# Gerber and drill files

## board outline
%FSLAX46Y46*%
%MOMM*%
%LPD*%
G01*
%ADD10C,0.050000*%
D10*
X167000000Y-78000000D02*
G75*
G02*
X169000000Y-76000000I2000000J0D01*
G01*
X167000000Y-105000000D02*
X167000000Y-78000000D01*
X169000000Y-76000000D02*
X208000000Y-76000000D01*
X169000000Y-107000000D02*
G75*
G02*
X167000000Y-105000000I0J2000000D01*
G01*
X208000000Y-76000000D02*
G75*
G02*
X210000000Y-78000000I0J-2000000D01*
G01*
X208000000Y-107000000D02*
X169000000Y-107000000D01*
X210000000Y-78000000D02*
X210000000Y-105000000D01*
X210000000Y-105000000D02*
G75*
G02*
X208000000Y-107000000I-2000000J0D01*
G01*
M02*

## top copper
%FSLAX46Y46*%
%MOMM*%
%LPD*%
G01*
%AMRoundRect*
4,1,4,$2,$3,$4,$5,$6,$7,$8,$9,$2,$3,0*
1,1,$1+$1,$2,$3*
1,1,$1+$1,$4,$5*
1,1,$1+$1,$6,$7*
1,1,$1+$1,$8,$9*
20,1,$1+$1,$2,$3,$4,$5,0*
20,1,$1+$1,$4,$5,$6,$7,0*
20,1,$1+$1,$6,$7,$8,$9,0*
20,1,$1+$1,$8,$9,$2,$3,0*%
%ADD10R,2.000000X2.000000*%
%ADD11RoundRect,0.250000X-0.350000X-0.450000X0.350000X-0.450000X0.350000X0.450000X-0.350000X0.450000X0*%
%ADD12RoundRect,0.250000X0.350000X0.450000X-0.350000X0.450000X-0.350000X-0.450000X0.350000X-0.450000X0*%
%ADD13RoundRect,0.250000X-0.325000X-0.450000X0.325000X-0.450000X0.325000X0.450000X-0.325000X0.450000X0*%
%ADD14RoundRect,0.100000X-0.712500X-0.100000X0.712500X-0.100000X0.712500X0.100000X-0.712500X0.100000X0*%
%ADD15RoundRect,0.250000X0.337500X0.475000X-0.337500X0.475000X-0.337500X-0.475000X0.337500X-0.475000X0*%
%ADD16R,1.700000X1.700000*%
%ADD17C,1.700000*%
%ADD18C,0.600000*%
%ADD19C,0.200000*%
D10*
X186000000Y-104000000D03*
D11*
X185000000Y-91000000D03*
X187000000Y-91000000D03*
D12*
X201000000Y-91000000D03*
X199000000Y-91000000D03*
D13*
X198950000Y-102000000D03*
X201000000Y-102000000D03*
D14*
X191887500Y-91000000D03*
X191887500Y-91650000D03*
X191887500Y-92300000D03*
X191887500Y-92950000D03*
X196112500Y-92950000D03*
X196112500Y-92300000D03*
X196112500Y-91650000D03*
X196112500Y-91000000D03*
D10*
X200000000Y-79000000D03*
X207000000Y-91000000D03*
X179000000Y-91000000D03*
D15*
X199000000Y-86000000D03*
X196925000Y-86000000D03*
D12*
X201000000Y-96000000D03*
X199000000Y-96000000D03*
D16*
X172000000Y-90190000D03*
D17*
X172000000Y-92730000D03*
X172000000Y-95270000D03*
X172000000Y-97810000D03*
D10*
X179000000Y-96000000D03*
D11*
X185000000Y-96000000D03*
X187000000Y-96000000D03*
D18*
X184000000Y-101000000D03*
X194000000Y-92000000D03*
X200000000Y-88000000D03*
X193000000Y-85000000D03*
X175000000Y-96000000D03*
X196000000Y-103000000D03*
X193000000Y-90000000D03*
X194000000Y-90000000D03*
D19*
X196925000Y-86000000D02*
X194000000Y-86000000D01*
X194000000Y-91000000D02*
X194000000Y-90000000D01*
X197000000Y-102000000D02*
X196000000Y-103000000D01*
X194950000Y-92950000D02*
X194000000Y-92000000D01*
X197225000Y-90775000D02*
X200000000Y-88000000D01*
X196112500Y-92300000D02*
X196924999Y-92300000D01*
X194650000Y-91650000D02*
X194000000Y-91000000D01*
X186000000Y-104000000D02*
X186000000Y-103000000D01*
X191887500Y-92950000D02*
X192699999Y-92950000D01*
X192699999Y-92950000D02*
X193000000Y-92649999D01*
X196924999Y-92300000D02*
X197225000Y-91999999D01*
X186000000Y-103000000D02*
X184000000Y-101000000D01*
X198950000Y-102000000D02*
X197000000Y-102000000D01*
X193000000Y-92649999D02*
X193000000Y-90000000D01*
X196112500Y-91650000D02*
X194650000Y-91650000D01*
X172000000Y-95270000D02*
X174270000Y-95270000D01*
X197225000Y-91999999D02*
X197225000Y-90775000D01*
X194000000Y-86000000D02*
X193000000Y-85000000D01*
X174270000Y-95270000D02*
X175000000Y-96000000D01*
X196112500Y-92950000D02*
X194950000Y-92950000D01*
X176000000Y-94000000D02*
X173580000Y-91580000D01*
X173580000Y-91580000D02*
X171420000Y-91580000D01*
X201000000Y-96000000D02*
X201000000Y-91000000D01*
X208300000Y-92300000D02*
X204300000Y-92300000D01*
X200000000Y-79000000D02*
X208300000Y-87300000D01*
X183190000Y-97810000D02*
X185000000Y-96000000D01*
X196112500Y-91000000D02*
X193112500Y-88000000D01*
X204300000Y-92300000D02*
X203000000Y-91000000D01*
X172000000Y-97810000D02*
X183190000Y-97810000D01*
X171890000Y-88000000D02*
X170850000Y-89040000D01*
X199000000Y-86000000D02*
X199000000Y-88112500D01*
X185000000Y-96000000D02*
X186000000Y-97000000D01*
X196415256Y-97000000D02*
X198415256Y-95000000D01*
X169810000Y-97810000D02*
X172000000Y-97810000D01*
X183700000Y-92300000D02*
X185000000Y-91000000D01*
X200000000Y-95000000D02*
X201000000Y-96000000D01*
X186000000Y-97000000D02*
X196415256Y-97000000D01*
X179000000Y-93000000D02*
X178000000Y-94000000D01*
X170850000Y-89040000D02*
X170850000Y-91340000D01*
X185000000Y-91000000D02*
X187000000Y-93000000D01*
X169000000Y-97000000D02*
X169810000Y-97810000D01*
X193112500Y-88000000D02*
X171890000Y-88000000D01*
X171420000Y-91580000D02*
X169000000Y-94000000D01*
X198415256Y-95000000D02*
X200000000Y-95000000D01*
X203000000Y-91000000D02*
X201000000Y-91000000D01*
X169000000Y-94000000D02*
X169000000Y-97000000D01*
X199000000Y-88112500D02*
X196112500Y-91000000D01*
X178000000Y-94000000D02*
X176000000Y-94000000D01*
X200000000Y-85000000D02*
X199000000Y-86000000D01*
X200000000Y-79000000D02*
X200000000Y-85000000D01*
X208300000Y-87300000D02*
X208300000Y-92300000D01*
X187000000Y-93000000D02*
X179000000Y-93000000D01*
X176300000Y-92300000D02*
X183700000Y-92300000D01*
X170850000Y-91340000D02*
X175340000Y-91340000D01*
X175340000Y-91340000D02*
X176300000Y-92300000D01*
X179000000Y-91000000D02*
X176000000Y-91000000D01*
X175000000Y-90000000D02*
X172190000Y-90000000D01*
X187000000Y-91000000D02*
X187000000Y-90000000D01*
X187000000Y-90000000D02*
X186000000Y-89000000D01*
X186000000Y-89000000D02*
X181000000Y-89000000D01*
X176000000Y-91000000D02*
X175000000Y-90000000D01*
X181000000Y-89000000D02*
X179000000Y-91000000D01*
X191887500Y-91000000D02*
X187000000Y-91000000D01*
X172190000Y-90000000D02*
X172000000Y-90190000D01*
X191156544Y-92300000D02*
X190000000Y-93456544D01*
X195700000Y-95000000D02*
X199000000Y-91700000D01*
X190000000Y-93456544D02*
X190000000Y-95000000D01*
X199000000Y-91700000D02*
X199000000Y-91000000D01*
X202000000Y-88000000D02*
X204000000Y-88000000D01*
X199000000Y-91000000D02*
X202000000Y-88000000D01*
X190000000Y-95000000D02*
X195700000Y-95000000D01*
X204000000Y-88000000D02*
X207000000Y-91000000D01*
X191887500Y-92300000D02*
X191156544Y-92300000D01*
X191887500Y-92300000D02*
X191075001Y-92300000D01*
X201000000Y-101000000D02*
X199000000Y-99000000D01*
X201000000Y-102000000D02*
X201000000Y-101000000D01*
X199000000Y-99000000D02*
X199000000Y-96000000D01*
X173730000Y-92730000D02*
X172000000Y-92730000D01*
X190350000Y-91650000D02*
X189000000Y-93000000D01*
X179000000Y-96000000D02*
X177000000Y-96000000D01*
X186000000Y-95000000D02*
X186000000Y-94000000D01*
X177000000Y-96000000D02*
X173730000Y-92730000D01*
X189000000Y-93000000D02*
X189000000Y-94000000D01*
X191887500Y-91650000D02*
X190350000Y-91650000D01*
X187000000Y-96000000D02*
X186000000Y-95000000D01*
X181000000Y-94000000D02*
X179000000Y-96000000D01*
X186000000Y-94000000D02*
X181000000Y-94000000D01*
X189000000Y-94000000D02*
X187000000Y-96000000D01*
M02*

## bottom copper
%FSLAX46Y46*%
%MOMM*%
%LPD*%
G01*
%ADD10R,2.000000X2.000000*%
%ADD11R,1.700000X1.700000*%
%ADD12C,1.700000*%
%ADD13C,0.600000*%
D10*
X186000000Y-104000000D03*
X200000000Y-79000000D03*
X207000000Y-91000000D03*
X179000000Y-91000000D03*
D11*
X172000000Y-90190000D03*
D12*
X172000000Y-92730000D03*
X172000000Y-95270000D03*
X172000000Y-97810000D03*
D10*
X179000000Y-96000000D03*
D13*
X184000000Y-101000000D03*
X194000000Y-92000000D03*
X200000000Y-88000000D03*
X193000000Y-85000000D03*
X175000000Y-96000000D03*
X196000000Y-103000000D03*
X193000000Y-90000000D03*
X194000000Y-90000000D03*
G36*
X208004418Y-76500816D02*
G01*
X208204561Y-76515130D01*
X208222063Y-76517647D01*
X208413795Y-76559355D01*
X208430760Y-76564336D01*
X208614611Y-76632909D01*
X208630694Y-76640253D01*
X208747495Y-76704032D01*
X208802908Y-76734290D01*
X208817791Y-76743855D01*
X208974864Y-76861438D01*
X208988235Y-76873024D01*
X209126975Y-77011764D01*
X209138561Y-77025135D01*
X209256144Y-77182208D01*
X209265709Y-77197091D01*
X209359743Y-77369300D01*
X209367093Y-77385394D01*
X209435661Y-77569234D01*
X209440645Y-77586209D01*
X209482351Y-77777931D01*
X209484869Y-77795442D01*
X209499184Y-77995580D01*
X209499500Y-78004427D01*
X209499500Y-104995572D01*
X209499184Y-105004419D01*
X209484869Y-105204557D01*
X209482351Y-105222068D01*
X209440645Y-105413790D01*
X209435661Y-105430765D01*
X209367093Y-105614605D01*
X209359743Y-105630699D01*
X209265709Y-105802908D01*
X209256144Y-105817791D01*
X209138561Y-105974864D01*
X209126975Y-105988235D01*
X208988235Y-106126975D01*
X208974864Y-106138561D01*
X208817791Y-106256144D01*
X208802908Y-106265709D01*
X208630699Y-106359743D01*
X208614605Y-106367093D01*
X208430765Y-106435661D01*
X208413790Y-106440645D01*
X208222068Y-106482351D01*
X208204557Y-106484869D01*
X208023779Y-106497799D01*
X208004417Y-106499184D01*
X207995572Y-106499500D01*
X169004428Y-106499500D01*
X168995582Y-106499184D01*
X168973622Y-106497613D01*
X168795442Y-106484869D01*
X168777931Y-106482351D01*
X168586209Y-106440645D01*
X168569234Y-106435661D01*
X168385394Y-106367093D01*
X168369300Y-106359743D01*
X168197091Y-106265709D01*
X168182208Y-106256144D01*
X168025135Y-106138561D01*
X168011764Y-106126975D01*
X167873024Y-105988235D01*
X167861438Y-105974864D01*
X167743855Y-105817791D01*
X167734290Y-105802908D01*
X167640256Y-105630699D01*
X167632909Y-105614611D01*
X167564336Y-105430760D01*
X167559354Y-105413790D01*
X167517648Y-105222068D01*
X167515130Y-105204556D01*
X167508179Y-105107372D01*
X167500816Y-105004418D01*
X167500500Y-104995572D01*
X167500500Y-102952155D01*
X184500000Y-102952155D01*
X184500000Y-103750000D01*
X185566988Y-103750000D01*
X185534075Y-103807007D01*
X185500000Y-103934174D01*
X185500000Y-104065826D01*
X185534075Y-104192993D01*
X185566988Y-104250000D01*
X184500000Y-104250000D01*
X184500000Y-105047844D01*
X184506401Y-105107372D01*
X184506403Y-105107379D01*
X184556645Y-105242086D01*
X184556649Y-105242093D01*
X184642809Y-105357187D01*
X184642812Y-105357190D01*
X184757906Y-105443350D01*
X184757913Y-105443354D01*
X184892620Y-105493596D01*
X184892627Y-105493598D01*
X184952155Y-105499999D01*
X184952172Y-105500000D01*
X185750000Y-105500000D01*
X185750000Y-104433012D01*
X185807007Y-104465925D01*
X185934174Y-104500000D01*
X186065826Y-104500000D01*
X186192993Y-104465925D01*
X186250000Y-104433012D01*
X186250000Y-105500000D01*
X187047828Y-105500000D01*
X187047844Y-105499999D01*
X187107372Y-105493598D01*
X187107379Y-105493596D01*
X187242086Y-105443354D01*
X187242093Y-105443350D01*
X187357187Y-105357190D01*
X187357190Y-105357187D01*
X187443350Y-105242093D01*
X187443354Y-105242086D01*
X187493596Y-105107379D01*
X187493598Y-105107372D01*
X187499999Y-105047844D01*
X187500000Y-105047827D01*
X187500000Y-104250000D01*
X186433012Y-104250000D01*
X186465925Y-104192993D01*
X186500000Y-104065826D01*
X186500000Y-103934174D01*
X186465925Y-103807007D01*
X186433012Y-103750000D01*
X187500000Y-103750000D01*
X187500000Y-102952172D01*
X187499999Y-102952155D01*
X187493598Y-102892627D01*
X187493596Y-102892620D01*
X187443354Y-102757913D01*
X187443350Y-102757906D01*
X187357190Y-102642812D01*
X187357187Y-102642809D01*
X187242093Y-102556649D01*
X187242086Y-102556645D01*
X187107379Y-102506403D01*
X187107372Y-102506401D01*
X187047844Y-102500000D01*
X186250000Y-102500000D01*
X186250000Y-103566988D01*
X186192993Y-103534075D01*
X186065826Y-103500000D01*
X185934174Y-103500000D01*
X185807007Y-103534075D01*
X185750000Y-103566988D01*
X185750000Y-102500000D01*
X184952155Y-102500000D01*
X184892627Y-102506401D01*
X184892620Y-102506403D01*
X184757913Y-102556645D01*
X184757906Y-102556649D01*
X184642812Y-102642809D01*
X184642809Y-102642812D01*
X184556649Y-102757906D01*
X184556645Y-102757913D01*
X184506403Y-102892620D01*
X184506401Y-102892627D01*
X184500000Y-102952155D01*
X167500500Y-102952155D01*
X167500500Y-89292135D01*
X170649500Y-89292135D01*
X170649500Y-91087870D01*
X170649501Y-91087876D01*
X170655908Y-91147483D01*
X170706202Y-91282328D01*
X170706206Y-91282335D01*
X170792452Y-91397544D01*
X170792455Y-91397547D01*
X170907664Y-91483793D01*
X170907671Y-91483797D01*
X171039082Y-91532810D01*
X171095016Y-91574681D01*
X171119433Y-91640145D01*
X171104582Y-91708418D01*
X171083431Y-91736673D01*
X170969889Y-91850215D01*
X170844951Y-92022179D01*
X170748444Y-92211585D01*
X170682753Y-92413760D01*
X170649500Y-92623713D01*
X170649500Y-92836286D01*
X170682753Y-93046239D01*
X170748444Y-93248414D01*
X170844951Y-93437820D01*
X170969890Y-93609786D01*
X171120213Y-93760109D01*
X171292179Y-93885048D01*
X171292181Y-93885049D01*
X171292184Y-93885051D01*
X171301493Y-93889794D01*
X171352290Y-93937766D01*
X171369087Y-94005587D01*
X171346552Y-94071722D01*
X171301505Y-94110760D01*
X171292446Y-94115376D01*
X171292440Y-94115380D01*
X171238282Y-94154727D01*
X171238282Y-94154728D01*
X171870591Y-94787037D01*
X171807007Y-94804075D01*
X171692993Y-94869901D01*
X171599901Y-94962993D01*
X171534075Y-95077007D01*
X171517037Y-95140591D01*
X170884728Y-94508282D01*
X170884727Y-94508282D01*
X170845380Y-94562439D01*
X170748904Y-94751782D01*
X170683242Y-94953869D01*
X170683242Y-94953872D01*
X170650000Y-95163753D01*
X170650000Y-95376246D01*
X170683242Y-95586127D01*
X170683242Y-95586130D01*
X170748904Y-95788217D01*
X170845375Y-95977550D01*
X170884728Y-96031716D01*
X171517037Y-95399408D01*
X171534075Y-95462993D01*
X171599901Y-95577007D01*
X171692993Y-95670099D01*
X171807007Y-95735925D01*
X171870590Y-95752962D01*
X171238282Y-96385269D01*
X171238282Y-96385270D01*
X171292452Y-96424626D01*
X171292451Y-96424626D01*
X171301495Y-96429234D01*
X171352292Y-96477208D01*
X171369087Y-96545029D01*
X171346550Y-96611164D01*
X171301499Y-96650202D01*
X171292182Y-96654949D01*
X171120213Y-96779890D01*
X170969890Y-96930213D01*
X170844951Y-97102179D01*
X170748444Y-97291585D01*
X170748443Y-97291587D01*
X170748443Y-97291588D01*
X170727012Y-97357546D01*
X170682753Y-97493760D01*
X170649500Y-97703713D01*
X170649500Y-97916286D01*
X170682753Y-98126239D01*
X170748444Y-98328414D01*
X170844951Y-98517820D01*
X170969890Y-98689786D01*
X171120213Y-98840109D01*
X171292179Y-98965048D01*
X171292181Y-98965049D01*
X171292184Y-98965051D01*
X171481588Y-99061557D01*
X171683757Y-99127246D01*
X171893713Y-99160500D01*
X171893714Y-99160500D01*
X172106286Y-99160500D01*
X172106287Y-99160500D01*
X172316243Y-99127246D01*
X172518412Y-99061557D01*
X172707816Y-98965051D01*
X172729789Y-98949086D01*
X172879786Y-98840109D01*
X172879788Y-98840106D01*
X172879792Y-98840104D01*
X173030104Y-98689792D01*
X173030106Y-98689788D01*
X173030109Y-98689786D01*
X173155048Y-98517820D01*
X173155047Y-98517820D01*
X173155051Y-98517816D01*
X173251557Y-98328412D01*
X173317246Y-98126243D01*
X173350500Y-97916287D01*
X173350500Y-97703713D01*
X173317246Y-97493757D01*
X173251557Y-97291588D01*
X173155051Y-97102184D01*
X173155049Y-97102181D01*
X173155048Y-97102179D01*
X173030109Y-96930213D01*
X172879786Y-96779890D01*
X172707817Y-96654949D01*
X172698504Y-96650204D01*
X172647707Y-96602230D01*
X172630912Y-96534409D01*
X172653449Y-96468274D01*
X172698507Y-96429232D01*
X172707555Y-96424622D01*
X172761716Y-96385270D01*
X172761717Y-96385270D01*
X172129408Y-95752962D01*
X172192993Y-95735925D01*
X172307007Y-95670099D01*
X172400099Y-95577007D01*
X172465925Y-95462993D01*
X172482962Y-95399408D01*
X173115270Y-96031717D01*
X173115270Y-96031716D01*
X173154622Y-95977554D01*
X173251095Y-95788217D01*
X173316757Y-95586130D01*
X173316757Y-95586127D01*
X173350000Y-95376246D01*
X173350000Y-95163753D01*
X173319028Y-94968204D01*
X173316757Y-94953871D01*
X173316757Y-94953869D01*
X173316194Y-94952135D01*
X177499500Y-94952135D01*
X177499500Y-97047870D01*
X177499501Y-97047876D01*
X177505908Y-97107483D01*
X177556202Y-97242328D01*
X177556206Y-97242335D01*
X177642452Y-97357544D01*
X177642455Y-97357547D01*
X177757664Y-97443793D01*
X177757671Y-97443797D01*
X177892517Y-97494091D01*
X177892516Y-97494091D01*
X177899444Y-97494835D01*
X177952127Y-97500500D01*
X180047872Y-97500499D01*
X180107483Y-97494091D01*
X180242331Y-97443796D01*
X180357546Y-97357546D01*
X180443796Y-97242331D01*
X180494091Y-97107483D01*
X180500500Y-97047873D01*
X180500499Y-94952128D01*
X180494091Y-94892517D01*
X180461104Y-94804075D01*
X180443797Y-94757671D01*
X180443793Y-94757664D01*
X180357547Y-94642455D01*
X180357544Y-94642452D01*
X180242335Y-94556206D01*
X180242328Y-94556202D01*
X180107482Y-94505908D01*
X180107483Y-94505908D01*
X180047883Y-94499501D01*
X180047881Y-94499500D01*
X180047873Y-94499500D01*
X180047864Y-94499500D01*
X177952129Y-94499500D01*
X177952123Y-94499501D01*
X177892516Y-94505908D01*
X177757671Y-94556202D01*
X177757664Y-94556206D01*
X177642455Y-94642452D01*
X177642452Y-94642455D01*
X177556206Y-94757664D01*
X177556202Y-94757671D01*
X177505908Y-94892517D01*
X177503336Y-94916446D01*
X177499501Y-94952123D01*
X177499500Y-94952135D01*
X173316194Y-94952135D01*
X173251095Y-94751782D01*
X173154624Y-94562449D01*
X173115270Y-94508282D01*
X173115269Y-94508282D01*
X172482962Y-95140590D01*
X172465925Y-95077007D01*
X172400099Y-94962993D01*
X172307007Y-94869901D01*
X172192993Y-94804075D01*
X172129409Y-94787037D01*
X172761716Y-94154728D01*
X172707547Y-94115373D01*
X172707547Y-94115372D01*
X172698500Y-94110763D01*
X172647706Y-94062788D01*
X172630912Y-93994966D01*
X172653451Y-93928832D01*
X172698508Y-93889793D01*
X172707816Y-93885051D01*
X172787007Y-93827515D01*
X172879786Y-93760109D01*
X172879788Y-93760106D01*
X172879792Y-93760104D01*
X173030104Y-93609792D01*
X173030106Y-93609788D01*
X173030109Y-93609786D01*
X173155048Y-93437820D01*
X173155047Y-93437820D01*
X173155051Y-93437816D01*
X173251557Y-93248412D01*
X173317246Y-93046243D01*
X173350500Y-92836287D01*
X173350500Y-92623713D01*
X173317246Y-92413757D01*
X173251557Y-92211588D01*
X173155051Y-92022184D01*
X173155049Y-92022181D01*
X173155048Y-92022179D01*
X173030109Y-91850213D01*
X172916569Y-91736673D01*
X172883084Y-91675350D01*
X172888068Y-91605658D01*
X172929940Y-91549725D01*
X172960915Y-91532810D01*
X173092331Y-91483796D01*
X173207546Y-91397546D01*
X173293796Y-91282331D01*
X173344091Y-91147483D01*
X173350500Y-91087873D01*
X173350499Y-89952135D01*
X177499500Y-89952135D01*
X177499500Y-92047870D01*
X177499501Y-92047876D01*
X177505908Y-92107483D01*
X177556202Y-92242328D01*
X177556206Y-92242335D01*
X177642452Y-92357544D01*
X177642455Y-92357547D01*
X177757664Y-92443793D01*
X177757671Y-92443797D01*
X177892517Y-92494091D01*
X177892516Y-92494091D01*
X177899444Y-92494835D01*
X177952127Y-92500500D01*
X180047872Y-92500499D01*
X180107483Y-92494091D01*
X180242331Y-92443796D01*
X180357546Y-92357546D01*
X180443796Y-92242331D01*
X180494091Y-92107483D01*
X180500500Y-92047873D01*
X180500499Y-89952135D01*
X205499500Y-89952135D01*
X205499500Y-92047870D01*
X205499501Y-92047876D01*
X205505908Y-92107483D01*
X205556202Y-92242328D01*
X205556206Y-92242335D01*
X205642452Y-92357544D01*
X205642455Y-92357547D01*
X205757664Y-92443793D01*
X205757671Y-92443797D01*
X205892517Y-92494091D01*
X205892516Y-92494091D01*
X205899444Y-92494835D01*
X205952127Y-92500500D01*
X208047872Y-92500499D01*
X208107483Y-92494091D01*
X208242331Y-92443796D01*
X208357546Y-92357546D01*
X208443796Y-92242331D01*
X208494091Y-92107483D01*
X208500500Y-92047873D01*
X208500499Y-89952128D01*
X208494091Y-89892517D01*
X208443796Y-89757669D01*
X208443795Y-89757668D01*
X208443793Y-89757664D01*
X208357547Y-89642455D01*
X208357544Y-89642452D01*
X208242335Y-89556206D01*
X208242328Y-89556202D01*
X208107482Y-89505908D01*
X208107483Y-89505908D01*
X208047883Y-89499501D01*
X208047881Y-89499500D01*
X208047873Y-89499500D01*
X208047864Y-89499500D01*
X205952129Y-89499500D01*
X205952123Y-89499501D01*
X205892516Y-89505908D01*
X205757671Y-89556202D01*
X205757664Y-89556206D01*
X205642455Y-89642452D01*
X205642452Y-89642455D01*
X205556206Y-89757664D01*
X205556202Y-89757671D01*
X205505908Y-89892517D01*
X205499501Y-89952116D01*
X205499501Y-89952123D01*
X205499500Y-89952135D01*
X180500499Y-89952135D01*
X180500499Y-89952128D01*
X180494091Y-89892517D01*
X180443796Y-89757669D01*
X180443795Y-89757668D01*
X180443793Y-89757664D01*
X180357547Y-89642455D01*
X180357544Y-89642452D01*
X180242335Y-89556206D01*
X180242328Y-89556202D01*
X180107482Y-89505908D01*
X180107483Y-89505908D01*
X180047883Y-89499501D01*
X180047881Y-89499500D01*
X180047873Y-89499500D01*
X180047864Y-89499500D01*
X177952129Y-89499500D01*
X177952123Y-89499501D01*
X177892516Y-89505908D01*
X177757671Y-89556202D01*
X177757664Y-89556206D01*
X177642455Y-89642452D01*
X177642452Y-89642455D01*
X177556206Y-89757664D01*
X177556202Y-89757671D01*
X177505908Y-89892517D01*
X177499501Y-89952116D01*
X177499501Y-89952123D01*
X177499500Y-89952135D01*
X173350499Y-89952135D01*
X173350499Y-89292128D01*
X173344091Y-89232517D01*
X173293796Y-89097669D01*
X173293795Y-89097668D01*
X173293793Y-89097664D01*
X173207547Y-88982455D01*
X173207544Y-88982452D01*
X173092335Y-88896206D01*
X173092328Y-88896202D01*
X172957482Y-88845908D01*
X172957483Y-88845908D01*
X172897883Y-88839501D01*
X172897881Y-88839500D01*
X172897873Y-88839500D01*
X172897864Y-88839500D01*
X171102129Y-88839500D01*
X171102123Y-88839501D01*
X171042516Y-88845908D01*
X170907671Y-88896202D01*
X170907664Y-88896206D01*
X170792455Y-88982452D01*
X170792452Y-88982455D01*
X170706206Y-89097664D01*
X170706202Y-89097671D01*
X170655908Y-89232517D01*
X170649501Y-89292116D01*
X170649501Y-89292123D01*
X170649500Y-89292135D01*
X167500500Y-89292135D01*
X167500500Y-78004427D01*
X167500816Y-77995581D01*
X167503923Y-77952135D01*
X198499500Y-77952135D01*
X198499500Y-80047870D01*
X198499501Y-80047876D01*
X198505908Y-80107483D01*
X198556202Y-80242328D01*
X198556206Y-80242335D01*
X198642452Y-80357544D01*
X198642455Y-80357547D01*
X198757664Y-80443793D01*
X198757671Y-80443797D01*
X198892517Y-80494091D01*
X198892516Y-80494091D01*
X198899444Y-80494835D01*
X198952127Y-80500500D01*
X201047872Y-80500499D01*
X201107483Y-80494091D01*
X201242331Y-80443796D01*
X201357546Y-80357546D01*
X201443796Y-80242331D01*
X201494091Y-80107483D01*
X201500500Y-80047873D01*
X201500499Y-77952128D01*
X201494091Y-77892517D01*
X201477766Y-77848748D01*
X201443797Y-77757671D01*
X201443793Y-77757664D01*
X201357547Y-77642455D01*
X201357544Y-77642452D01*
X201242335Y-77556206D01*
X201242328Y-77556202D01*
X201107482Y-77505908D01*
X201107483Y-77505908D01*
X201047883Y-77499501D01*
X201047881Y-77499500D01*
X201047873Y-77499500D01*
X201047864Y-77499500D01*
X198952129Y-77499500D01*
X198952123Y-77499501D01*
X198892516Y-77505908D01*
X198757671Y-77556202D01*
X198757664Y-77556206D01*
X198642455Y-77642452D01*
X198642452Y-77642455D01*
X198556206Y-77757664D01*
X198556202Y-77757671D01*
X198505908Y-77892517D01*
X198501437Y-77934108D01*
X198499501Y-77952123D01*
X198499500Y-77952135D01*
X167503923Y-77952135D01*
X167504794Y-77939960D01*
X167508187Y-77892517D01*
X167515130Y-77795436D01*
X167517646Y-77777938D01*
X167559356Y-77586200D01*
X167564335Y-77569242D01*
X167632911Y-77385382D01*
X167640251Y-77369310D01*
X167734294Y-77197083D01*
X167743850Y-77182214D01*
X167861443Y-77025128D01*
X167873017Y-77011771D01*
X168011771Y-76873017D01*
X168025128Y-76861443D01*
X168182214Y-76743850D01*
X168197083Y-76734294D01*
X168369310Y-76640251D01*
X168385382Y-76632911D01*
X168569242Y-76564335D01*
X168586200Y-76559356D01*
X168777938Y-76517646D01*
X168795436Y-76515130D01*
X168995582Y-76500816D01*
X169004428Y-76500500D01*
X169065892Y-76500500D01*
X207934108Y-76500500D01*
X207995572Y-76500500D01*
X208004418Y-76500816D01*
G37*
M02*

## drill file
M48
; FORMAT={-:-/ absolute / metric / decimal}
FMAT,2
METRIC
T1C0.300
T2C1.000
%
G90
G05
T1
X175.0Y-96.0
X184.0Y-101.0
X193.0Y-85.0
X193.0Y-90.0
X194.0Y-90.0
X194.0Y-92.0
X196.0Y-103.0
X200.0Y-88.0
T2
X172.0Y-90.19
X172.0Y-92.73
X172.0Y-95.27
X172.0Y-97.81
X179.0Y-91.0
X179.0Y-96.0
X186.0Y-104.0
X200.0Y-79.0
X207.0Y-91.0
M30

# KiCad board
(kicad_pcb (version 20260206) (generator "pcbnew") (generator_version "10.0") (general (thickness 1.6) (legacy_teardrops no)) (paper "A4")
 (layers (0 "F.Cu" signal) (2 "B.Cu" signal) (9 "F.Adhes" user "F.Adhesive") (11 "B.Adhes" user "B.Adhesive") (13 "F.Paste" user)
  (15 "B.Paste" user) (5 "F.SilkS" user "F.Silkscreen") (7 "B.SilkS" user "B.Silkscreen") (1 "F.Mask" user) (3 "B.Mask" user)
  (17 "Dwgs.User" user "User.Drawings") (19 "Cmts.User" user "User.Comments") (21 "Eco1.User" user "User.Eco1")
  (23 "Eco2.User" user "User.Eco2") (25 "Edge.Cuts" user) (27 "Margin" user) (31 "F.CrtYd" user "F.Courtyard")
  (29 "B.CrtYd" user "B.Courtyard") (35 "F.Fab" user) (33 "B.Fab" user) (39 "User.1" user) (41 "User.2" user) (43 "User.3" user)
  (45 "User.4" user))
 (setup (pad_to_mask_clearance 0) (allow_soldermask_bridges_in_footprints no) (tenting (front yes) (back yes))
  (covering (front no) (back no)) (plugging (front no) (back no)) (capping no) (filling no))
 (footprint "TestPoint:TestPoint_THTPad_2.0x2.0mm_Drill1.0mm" (layer "F.Cu") (at 186 104)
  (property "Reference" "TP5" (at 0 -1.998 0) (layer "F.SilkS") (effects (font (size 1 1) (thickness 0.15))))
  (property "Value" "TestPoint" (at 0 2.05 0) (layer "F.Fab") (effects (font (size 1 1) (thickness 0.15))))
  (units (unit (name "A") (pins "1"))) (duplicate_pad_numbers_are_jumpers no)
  (pad "1" thru_hole rect (at 0 0) (size 2 2) (drill 1) (layers "*.Cu" "*.Mask") (remove_unused_layers no) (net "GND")))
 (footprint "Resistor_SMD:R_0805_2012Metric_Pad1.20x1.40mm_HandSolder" (layer "F.Cu") (at 186 91)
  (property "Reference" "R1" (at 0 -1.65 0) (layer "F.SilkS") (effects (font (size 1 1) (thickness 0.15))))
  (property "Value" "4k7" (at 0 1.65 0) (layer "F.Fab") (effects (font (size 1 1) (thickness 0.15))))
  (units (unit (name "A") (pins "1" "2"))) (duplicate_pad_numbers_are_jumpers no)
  (pad "1" smd roundrect (at -1 0) (size 1.2 1.4) (layers "F.Cu" "F.Mask" "F.Paste") (roundrect_rratio 0.208333) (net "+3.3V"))
  (pad "2" smd roundrect (at 1 0) (size 1.2 1.4) (layers "F.Cu" "F.Mask" "F.Paste") (roundrect_rratio 0.208333) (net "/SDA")))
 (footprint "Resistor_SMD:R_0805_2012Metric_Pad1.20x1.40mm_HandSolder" (layer "F.Cu") (at 200 91 180)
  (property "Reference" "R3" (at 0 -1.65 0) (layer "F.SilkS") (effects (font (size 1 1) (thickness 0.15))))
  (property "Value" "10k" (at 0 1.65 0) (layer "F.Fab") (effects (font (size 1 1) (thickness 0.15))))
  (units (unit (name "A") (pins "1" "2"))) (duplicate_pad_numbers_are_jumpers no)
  (pad "1" smd roundrect (at -1 0 180) (size 1.2 1.4) (layers "F.Cu" "F.Mask" "F.Paste") (roundrect_rratio 0.208333) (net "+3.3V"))
  (pad "2" smd roundrect (at 1 0 180) (size 1.2 1.4) (layers "F.Cu" "F.Mask" "F.Paste") (roundrect_rratio 0.208333) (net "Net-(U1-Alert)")))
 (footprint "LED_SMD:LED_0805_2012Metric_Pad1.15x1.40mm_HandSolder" (layer "F.Cu") (at 199.975 102)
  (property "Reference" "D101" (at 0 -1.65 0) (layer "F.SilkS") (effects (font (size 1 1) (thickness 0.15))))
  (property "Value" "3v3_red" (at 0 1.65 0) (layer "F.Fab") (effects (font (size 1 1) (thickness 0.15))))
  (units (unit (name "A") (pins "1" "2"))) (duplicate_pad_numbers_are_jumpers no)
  (pad "1" smd roundrect (at -1.025 0) (size 1.15 1.4) (layers "F.Cu" "F.Mask" "F.Paste") (roundrect_rratio 0.217391) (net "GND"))
  (pad "2" smd roundrect (at 1.025 0) (size 1.15 1.4) (layers "F.Cu" "F.Mask" "F.Paste") (roundrect_rratio 0.217391) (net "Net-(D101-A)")))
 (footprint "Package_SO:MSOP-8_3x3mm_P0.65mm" (layer "F.Cu") (at 194 91.975)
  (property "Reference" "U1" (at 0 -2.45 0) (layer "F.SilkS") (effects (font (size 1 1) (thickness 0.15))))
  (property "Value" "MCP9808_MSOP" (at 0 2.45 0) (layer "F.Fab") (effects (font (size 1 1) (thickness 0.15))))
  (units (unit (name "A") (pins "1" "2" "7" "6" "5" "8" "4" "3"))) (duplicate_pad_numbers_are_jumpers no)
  (pad "1" smd roundrect (at -2.1125 -0.975) (size 1.625 0.4) (layers "F.Cu" "F.Mask" "F.Paste") (roundrect_rratio 0.25) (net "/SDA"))
  (pad "2" smd roundrect (at -2.1125 -0.325) (size 1.625 0.4) (layers "F.Cu" "F.Mask" "F.Paste") (roundrect_rratio 0.25) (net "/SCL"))
  (pad "3" smd roundrect (at -2.1125 0.325) (size 1.625 0.4) (layers "F.Cu" "F.Mask" "F.Paste") (roundrect_rratio 0.25)
   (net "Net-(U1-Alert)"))
  (pad "4" smd roundrect (at -2.1125 0.975) (size 1.625 0.4) (layers "F.Cu" "F.Mask" "F.Paste") (roundrect_rratio 0.25) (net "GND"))
  (pad "5" smd roundrect (at 2.1125 0.975) (size 1.625 0.4) (layers "F.Cu" "F.Mask" "F.Paste") (roundrect_rratio 0.25) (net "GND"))
  (pad "6" smd roundrect (at 2.1125 0.325) (size 1.625 0.4) (layers "F.Cu" "F.Mask" "F.Paste") (roundrect_rratio 0.25) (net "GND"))
  (pad "7" smd roundrect (at 2.1125 -0.325) (size 1.625 0.4) (layers "F.Cu" "F.Mask" "F.Paste") (roundrect_rratio 0.25) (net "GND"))
  (pad "8" smd roundrect (at 2.1125 -0.975) (size 1.625 0.4) (layers "F.Cu" "F.Mask" "F.Paste") (roundrect_rratio 0.25) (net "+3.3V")))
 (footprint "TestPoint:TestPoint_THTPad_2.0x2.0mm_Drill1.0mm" (layer "F.Cu") (at 200 79)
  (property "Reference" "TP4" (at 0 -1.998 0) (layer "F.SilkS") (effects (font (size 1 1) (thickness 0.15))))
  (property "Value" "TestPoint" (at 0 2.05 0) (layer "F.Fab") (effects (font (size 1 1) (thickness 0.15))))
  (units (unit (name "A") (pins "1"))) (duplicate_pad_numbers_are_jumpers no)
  (pad "1" thru_hole rect (at 0 0) (size 2 2) (drill 1) (layers "*.Cu" "*.Mask") (remove_unused_layers no) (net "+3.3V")))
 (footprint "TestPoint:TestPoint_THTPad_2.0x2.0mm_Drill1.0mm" (layer "F.Cu") (at 207 91)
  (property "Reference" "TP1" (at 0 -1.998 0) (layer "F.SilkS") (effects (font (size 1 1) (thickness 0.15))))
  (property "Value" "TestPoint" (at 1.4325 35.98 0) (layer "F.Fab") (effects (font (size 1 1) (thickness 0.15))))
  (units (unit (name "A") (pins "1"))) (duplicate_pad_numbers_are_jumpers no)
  (pad "1" thru_hole rect (at 0 0) (size 2 2) (drill 1) (layers "*.Cu" "*.Mask") (remove_unused_layers no) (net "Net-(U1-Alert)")))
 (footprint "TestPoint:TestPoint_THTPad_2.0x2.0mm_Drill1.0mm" (layer "F.Cu") (at 179 91)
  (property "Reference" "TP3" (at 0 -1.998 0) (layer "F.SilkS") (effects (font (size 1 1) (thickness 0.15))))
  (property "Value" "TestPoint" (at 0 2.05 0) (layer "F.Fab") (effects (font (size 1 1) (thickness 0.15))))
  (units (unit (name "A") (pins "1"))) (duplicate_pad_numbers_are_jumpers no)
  (pad "1" thru_hole rect (at 0 0) (size 2 2) (drill 1) (layers "*.Cu" "*.Mask") (remove_unused_layers no) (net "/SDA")))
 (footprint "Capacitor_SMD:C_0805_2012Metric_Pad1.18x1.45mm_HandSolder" (layer "F.Cu") (at 197.9625 86 180)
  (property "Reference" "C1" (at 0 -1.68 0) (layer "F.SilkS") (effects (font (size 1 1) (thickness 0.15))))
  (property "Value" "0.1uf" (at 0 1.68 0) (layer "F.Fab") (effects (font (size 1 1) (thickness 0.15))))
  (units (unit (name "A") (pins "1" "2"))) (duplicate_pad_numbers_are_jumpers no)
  (pad "1" smd roundrect (at -1.0375 0 180) (size 1.175 1.45) (layers "F.Cu" "F.Mask" "F.Paste") (roundrect_rratio 0.212766) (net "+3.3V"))
  (pad "2" smd roundrect (at 1.0375 0 180) (size 1.175 1.45) (layers "F.Cu" "F.Mask" "F.Paste") (roundrect_rratio 0.212766) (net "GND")))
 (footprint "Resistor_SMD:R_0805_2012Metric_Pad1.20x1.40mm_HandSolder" (layer "F.Cu") (at 200 96 180)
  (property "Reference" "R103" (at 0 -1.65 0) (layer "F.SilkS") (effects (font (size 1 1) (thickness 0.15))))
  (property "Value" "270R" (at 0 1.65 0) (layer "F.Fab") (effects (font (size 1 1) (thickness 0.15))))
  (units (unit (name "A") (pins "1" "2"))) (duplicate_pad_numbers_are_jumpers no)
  (pad "1" smd roundrect (at -1 0 180) (size 1.2 1.4) (layers "F.Cu" "F.Mask" "F.Paste") (roundrect_rratio 0.208333) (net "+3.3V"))
  (pad "2" smd roundrect (at 1 0 180) (size 1.2 1.4) (layers "F.Cu" "F.Mask" "F.Paste") (roundrect_rratio 0.208333) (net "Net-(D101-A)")))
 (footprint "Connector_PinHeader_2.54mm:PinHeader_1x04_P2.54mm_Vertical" (layer "F.Cu") (at 172 90.19)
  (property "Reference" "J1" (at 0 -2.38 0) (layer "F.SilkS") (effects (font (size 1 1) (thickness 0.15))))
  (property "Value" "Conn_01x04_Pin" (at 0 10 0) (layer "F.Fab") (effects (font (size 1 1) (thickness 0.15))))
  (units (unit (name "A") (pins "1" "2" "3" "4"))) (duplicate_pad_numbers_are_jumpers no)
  (pad "1" thru_hole rect (at 0 0) (size 1.7 1.7) (drill 1) (layers "*.Cu" "*.Mask") (remove_unused_layers no) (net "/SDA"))
  (pad "2" thru_hole circle (at 0 2.54) (size 1.7 1.7) (drill 1) (layers "*.Cu" "*.Mask") (remove_unused_layers no) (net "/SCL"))
  (pad "3" thru_hole circle (at 0 5.08) (size 1.7 1.7) (drill 1) (layers "*.Cu" "*.Mask") (remove_unused_layers no) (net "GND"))
  (pad "4" thru_hole circle (at 0 7.62) (size 1.7 1.7) (drill 1) (layers "*.Cu" "*.Mask") (remove_unused_layers no) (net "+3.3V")))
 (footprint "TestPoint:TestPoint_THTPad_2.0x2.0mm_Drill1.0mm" (layer "F.Cu") (at 179 96)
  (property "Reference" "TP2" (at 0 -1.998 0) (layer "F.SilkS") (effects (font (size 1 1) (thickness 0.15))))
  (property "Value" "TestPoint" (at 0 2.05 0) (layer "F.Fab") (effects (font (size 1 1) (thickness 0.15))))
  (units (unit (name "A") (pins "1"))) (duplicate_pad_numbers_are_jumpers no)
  (pad "1" thru_hole rect (at 0 0) (size 2 2) (drill 1) (layers "*.Cu" "*.Mask") (remove_unused_layers no) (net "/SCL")))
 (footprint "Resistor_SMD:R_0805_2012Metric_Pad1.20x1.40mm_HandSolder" (layer "F.Cu") (at 186 96)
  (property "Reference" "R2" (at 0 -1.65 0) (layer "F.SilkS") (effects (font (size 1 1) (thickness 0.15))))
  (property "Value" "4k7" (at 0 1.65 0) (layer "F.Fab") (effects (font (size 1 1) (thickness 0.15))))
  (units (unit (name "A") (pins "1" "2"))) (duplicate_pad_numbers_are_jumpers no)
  (pad "1" smd roundrect (at -1 0) (size 1.2 1.4) (layers "F.Cu" "F.Mask" "F.Paste") (roundrect_rratio 0.208333) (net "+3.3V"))
  (pad "2" smd roundrect (at 1 0) (size 1.2 1.4) (layers "F.Cu" "F.Mask" "F.Paste") (roundrect_rratio 0.208333) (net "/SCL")))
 (gr_arc (start 167 78) (mid 167.585786 76.585786) (end 169 76) (stroke (width 0.05) (type default)) (layer "Edge.Cuts"))
 (gr_line (start 167 105) (end 167 78) (stroke (width 0.05) (type default)) (layer "Edge.Cuts"))
 (gr_line (start 169 76) (end 208 76) (stroke (width 0.05) (type default)) (layer "Edge.Cuts"))
 (gr_arc (start 169 107) (mid 167.585786 106.414214) (end 167 105) (stroke (width 0.05) (type default)) (layer "Edge.Cuts"))
 (gr_arc (start 208 76) (mid 209.414214 76.585786) (end 210 78) (stroke (width 0.05) (type default)) (layer "Edge.Cuts"))
 (gr_line (start 208 107) (end 169 107) (stroke (width 0.05) (type default)) (layer "Edge.Cuts"))
 (gr_line (start 210 78) (end 210 105) (stroke (width 0.05) (type default)) (layer "Edge.Cuts"))
 (gr_arc (start 210 105) (mid 209.414214 106.414214) (end 208 107) (stroke (width 0.05) (type default)) (layer "Edge.Cuts"))
 (segment (start 196.925 86) (end 194 86) (width 0.2) (layer "F.Cu") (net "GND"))
 (segment (start 194 91) (end 194 90) (width 0.2) (layer "F.Cu") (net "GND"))
 (segment (start 197 102) (end 196 103) (width 0.2) (layer "F.Cu") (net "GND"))
 (segment (start 194.95 92.95) (end 194 92) (width 0.2) (layer "F.Cu") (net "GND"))
 (segment (start 197.225 90.775) (end 200 88) (width 0.2) (layer "F.Cu") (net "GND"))
 (segment (start 196.1125 92.3) (end 196.924999 92.3) (width 0.2) (layer "F.Cu") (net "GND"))
 (segment (start 194.65 91.65) (end 194 91) (width 0.2) (layer "F.Cu") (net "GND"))
 (segment (start 186 104) (end 186 103) (width 0.2) (layer "F.Cu") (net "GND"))
 (segment (start 191.8875 92.95) (end 192.699999 92.95) (width 0.2) (layer "F.Cu") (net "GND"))
 (segment (start 192.699999 92.95) (end 193 92.649999) (width 0.2) (layer "F.Cu") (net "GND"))
 (segment (start 196.924999 92.3) (end 197.225 91.999999) (width 0.2) (layer "F.Cu") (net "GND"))
 (segment (start 186 103) (end 184 101) (width 0.2) (layer "F.Cu") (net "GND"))
 (segment (start 198.95 102) (end 197 102) (width 0.2) (layer "F.Cu") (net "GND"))
 (segment (start 193 92.649999) (end 193 90) (width 0.2) (layer "F.Cu") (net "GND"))
 (segment (start 196.1125 91.65) (end 194.65 91.65) (width 0.2) (layer "F.Cu") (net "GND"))
 (segment (start 172 95.27) (end 174.27 95.27) (width 0.2) (layer "F.Cu") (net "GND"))
 (segment (start 197.225 91.999999) (end 197.225 90.775) (width 0.2) (layer "F.Cu") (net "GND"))
 (segment (start 194 86) (end 193 85) (width 0.2) (layer "F.Cu") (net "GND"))
 (segment (start 174.27 95.27) (end 175 96) (width 0.2) (layer "F.Cu") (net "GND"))
 (segment (start 196.1125 92.95) (end 194.95 92.95) (width 0.2) (layer "F.Cu") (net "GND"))
 (via (at 184 101) (size 0.6) (drill 0.3) (layers "F.Cu" "B.Cu") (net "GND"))
 (via (at 194 92) (size 0.6) (drill 0.3) (layers "F.Cu" "B.Cu") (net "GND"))
 (via (at 200 88) (size 0.6) (drill 0.3) (layers "F.Cu" "B.Cu") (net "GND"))
 (via (at 193 85) (size 0.6) (drill 0.3) (layers "F.Cu" "B.Cu") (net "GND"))
 (via (at 175 96) (size 0.6) (drill 0.3) (layers "F.Cu" "B.Cu") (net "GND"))
 (via (at 196 103) (size 0.6) (drill 0.3) (layers "F.Cu" "B.Cu") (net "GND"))
 (via (at 193 90) (size 0.6) (drill 0.3) (layers "F.Cu" "B.Cu") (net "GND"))
 (via (at 194 90) (size 0.6) (drill 0.3) (layers "F.Cu" "B.Cu") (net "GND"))
 (segment (start 176 94) (end 173.58 91.58) (width 0.2) (layer "F.Cu") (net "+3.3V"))
 (segment (start 173.58 91.58) (end 171.42 91.58) (width 0.2) (layer "F.Cu") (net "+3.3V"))
 (segment (start 201 96) (end 201 91) (width 0.2) (layer "F.Cu") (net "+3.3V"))
 (segment (start 208.3 92.3) (end 204.3 92.3) (width 0.2) (layer "F.Cu") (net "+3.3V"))
 (segment (start 200 79) (end 208.3 87.3) (width 0.2) (layer "F.Cu") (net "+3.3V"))
 (segment (start 183.19 97.81) (end 185 96) (width 0.2) (layer "F.Cu") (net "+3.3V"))
 (segment (start 196.1125 91) (end 193.1125 88) (width 0.2) (layer "F.Cu") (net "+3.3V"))
 (segment (start 204.3 92.3) (end 203 91) (width 0.2) (layer "F.Cu") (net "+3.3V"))
 (segment (start 172 97.81) (end 183.19 97.81) (width 0.2) (layer "F.Cu") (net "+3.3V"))
 (segment (start 171.89 88) (end 170.85 89.04) (width 0.2) (layer "F.Cu") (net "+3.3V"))
 (segment (start 199 86) (end 199 88.1125) (width 0.2) (layer "F.Cu") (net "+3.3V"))
 (segment (start 185 96) (end 186 97) (width 0.2) (layer "F.Cu") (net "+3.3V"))
 (segment (start 196.415256 97) (end 198.415256 95) (width 0.2) (layer "F.Cu") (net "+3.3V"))
 (segment (start 169.81 97.81) (end 172 97.81) (width 0.2) (layer "F.Cu") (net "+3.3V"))
 (segment (start 183.7 92.3) (end 185 91) (width 0.2) (layer "F.Cu") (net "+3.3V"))
 (segment (start 200 95) (end 201 96) (width 0.2) (layer "F.Cu") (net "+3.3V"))
 (segment (start 186 97) (end 196.415256 97) (width 0.2) (layer "F.Cu") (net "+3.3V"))
 (segment (start 179 93) (end 178 94) (width 0.2) (layer "F.Cu") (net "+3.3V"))
 (segment (start 170.85 89.04) (end 170.85 91.34) (width 0.2) (layer "F.Cu") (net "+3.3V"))
 (segment (start 185 91) (end 187 93) (width 0.2) (layer "F.Cu") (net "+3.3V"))
 (segment (start 169 97) (end 169.81 97.81) (width 0.2) (layer "F.Cu") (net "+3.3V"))
 (segment (start 193.1125 88) (end 171.89 88) (width 0.2) (layer "F.Cu") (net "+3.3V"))
 (segment (start 171.42 91.58) (end 169 94) (width 0.2) (layer "F.Cu") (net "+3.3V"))
 (segment (start 198.415256 95) (end 200 95) (width 0.2) (layer "F.Cu") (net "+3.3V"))
 (segment (start 203 91) (end 201 91) (width 0.2) (layer "F.Cu") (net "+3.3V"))
 (segment (start 169 94) (end 169 97) (width 0.2) (layer "F.Cu") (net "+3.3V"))
 (segment (start 199 88.1125) (end 196.1125 91) (width 0.2) (layer "F.Cu") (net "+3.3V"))
 (segment (start 178 94) (end 176 94) (width 0.2) (layer "F.Cu") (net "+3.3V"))
 (segment (start 200 85) (end 199 86) (width 0.2) (layer "F.Cu") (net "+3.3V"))
 (segment (start 200 79) (end 200 85) (width 0.2) (layer "F.Cu") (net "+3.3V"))
 (segment (start 208.3 87.3) (end 208.3 92.3) (width 0.2) (layer "F.Cu") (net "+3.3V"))
 (segment (start 187 93) (end 179 93) (width 0.2) (layer "F.Cu") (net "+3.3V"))
 (segment (start 176.3 92.3) (end 183.7 92.3) (width 0.2) (layer "F.Cu") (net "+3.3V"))
 (segment (start 170.85 91.34) (end 175.34 91.34) (width 0.2) (layer "F.Cu") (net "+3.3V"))
 (segment (start 175.34 91.34) (end 176.3 92.3) (width 0.2) (layer "F.Cu") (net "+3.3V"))
 (segment (start 179 91) (end 176 91) (width 0.2) (layer "F.Cu") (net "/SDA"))
 (segment (start 175 90) (end 172.19 90) (width 0.2) (layer "F.Cu") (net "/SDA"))
 (segment (start 187 91) (end 187 90) (width 0.2) (layer "F.Cu") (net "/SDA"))
 (segment (start 187 90) (end 186 89) (width 0.2) (layer "F.Cu") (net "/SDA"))
 (segment (start 186 89) (end 181 89) (width 0.2) (layer "F.Cu") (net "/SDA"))
 (segment (start 176 91) (end 175 90) (width 0.2) (layer "F.Cu") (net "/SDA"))
 (segment (start 181 89) (end 179 91) (width 0.2) (layer "F.Cu") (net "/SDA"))
 (segment (start 191.8875 91) (end 187 91) (width 0.2) (layer "F.Cu") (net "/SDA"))
 (segment (start 172.19 90) (end 172 90.19) (width 0.2) (layer "F.Cu") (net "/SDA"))
 (segment (start 191.156544 92.3) (end 190 93.456544) (width 0.2) (layer "F.Cu") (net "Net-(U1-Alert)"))
 (segment (start 195.7 95) (end 199 91.7) (width 0.2) (layer "F.Cu") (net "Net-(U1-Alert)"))
 (segment (start 190 93.456544) (end 190 95) (width 0.2) (layer "F.Cu") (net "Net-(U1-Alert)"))
 (segment (start 199 91.7) (end 199 91) (width 0.2) (layer "F.Cu") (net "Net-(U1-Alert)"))
 (segment (start 202 88) (end 204 88) (width 0.2) (layer "F.Cu") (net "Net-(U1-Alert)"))
 (segment (start 199 91) (end 202 88) (width 0.2) (layer "F.Cu") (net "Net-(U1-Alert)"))
 (segment (start 190 95) (end 195.7 95) (width 0.2) (layer "F.Cu") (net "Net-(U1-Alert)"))
 (segment (start 204 88) (end 207 91) (width 0.2) (layer "F.Cu") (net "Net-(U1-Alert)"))
 (segment (start 191.8875 92.3) (end 191.156544 92.3) (width 0.2) (layer "F.Cu") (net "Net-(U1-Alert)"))
 (segment (start 191.8875 92.3) (end 191.075001 92.3) (width 0.2) (layer "F.Cu") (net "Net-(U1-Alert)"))
 (segment (start 201 101) (end 199 99) (width 0.2) (layer "F.Cu") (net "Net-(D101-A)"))
 (segment (start 201 102) (end 201 101) (width 0.2) (layer "F.Cu") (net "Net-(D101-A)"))
 (segment (start 199 99) (end 199 96) (width 0.2) (layer "F.Cu") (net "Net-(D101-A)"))
 (segment (start 173.73 92.73) (end 172 92.73) (width 0.2) (layer "F.Cu") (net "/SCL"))
 (segment (start 190.35 91.65) (end 189 93) (width 0.2) (layer "F.Cu") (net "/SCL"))
 (segment (start 179 96) (end 177 96) (width 0.2) (layer "F.Cu") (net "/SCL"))
 (segment (start 186 95) (end 186 94) (width 0.2) (layer "F.Cu") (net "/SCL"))
 (segment (start 177 96) (end 173.73 92.73) (width 0.2) (layer "F.Cu") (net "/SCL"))
 (segment (start 189 93) (end 189 94) (width 0.2) (layer "F.Cu") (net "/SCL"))
 (segment (start 191.8875 91.65) (end 190.35 91.65) (width 0.2) (layer "F.Cu") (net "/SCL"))
 (segment (start 187 96) (end 186 95) (width 0.2) (layer "F.Cu") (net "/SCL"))
 (segment (start 181 94) (end 179 96) (width 0.2) (layer "F.Cu") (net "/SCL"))
 (segment (start 186 94) (end 181 94) (width 0.2) (layer "F.Cu") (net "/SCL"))
 (segment (start 189 94) (end 187 96) (width 0.2) (layer "F.Cu") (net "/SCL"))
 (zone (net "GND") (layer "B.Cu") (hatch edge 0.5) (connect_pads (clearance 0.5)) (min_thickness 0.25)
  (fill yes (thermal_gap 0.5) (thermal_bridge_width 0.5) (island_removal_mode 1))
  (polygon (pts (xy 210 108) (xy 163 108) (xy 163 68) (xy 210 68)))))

